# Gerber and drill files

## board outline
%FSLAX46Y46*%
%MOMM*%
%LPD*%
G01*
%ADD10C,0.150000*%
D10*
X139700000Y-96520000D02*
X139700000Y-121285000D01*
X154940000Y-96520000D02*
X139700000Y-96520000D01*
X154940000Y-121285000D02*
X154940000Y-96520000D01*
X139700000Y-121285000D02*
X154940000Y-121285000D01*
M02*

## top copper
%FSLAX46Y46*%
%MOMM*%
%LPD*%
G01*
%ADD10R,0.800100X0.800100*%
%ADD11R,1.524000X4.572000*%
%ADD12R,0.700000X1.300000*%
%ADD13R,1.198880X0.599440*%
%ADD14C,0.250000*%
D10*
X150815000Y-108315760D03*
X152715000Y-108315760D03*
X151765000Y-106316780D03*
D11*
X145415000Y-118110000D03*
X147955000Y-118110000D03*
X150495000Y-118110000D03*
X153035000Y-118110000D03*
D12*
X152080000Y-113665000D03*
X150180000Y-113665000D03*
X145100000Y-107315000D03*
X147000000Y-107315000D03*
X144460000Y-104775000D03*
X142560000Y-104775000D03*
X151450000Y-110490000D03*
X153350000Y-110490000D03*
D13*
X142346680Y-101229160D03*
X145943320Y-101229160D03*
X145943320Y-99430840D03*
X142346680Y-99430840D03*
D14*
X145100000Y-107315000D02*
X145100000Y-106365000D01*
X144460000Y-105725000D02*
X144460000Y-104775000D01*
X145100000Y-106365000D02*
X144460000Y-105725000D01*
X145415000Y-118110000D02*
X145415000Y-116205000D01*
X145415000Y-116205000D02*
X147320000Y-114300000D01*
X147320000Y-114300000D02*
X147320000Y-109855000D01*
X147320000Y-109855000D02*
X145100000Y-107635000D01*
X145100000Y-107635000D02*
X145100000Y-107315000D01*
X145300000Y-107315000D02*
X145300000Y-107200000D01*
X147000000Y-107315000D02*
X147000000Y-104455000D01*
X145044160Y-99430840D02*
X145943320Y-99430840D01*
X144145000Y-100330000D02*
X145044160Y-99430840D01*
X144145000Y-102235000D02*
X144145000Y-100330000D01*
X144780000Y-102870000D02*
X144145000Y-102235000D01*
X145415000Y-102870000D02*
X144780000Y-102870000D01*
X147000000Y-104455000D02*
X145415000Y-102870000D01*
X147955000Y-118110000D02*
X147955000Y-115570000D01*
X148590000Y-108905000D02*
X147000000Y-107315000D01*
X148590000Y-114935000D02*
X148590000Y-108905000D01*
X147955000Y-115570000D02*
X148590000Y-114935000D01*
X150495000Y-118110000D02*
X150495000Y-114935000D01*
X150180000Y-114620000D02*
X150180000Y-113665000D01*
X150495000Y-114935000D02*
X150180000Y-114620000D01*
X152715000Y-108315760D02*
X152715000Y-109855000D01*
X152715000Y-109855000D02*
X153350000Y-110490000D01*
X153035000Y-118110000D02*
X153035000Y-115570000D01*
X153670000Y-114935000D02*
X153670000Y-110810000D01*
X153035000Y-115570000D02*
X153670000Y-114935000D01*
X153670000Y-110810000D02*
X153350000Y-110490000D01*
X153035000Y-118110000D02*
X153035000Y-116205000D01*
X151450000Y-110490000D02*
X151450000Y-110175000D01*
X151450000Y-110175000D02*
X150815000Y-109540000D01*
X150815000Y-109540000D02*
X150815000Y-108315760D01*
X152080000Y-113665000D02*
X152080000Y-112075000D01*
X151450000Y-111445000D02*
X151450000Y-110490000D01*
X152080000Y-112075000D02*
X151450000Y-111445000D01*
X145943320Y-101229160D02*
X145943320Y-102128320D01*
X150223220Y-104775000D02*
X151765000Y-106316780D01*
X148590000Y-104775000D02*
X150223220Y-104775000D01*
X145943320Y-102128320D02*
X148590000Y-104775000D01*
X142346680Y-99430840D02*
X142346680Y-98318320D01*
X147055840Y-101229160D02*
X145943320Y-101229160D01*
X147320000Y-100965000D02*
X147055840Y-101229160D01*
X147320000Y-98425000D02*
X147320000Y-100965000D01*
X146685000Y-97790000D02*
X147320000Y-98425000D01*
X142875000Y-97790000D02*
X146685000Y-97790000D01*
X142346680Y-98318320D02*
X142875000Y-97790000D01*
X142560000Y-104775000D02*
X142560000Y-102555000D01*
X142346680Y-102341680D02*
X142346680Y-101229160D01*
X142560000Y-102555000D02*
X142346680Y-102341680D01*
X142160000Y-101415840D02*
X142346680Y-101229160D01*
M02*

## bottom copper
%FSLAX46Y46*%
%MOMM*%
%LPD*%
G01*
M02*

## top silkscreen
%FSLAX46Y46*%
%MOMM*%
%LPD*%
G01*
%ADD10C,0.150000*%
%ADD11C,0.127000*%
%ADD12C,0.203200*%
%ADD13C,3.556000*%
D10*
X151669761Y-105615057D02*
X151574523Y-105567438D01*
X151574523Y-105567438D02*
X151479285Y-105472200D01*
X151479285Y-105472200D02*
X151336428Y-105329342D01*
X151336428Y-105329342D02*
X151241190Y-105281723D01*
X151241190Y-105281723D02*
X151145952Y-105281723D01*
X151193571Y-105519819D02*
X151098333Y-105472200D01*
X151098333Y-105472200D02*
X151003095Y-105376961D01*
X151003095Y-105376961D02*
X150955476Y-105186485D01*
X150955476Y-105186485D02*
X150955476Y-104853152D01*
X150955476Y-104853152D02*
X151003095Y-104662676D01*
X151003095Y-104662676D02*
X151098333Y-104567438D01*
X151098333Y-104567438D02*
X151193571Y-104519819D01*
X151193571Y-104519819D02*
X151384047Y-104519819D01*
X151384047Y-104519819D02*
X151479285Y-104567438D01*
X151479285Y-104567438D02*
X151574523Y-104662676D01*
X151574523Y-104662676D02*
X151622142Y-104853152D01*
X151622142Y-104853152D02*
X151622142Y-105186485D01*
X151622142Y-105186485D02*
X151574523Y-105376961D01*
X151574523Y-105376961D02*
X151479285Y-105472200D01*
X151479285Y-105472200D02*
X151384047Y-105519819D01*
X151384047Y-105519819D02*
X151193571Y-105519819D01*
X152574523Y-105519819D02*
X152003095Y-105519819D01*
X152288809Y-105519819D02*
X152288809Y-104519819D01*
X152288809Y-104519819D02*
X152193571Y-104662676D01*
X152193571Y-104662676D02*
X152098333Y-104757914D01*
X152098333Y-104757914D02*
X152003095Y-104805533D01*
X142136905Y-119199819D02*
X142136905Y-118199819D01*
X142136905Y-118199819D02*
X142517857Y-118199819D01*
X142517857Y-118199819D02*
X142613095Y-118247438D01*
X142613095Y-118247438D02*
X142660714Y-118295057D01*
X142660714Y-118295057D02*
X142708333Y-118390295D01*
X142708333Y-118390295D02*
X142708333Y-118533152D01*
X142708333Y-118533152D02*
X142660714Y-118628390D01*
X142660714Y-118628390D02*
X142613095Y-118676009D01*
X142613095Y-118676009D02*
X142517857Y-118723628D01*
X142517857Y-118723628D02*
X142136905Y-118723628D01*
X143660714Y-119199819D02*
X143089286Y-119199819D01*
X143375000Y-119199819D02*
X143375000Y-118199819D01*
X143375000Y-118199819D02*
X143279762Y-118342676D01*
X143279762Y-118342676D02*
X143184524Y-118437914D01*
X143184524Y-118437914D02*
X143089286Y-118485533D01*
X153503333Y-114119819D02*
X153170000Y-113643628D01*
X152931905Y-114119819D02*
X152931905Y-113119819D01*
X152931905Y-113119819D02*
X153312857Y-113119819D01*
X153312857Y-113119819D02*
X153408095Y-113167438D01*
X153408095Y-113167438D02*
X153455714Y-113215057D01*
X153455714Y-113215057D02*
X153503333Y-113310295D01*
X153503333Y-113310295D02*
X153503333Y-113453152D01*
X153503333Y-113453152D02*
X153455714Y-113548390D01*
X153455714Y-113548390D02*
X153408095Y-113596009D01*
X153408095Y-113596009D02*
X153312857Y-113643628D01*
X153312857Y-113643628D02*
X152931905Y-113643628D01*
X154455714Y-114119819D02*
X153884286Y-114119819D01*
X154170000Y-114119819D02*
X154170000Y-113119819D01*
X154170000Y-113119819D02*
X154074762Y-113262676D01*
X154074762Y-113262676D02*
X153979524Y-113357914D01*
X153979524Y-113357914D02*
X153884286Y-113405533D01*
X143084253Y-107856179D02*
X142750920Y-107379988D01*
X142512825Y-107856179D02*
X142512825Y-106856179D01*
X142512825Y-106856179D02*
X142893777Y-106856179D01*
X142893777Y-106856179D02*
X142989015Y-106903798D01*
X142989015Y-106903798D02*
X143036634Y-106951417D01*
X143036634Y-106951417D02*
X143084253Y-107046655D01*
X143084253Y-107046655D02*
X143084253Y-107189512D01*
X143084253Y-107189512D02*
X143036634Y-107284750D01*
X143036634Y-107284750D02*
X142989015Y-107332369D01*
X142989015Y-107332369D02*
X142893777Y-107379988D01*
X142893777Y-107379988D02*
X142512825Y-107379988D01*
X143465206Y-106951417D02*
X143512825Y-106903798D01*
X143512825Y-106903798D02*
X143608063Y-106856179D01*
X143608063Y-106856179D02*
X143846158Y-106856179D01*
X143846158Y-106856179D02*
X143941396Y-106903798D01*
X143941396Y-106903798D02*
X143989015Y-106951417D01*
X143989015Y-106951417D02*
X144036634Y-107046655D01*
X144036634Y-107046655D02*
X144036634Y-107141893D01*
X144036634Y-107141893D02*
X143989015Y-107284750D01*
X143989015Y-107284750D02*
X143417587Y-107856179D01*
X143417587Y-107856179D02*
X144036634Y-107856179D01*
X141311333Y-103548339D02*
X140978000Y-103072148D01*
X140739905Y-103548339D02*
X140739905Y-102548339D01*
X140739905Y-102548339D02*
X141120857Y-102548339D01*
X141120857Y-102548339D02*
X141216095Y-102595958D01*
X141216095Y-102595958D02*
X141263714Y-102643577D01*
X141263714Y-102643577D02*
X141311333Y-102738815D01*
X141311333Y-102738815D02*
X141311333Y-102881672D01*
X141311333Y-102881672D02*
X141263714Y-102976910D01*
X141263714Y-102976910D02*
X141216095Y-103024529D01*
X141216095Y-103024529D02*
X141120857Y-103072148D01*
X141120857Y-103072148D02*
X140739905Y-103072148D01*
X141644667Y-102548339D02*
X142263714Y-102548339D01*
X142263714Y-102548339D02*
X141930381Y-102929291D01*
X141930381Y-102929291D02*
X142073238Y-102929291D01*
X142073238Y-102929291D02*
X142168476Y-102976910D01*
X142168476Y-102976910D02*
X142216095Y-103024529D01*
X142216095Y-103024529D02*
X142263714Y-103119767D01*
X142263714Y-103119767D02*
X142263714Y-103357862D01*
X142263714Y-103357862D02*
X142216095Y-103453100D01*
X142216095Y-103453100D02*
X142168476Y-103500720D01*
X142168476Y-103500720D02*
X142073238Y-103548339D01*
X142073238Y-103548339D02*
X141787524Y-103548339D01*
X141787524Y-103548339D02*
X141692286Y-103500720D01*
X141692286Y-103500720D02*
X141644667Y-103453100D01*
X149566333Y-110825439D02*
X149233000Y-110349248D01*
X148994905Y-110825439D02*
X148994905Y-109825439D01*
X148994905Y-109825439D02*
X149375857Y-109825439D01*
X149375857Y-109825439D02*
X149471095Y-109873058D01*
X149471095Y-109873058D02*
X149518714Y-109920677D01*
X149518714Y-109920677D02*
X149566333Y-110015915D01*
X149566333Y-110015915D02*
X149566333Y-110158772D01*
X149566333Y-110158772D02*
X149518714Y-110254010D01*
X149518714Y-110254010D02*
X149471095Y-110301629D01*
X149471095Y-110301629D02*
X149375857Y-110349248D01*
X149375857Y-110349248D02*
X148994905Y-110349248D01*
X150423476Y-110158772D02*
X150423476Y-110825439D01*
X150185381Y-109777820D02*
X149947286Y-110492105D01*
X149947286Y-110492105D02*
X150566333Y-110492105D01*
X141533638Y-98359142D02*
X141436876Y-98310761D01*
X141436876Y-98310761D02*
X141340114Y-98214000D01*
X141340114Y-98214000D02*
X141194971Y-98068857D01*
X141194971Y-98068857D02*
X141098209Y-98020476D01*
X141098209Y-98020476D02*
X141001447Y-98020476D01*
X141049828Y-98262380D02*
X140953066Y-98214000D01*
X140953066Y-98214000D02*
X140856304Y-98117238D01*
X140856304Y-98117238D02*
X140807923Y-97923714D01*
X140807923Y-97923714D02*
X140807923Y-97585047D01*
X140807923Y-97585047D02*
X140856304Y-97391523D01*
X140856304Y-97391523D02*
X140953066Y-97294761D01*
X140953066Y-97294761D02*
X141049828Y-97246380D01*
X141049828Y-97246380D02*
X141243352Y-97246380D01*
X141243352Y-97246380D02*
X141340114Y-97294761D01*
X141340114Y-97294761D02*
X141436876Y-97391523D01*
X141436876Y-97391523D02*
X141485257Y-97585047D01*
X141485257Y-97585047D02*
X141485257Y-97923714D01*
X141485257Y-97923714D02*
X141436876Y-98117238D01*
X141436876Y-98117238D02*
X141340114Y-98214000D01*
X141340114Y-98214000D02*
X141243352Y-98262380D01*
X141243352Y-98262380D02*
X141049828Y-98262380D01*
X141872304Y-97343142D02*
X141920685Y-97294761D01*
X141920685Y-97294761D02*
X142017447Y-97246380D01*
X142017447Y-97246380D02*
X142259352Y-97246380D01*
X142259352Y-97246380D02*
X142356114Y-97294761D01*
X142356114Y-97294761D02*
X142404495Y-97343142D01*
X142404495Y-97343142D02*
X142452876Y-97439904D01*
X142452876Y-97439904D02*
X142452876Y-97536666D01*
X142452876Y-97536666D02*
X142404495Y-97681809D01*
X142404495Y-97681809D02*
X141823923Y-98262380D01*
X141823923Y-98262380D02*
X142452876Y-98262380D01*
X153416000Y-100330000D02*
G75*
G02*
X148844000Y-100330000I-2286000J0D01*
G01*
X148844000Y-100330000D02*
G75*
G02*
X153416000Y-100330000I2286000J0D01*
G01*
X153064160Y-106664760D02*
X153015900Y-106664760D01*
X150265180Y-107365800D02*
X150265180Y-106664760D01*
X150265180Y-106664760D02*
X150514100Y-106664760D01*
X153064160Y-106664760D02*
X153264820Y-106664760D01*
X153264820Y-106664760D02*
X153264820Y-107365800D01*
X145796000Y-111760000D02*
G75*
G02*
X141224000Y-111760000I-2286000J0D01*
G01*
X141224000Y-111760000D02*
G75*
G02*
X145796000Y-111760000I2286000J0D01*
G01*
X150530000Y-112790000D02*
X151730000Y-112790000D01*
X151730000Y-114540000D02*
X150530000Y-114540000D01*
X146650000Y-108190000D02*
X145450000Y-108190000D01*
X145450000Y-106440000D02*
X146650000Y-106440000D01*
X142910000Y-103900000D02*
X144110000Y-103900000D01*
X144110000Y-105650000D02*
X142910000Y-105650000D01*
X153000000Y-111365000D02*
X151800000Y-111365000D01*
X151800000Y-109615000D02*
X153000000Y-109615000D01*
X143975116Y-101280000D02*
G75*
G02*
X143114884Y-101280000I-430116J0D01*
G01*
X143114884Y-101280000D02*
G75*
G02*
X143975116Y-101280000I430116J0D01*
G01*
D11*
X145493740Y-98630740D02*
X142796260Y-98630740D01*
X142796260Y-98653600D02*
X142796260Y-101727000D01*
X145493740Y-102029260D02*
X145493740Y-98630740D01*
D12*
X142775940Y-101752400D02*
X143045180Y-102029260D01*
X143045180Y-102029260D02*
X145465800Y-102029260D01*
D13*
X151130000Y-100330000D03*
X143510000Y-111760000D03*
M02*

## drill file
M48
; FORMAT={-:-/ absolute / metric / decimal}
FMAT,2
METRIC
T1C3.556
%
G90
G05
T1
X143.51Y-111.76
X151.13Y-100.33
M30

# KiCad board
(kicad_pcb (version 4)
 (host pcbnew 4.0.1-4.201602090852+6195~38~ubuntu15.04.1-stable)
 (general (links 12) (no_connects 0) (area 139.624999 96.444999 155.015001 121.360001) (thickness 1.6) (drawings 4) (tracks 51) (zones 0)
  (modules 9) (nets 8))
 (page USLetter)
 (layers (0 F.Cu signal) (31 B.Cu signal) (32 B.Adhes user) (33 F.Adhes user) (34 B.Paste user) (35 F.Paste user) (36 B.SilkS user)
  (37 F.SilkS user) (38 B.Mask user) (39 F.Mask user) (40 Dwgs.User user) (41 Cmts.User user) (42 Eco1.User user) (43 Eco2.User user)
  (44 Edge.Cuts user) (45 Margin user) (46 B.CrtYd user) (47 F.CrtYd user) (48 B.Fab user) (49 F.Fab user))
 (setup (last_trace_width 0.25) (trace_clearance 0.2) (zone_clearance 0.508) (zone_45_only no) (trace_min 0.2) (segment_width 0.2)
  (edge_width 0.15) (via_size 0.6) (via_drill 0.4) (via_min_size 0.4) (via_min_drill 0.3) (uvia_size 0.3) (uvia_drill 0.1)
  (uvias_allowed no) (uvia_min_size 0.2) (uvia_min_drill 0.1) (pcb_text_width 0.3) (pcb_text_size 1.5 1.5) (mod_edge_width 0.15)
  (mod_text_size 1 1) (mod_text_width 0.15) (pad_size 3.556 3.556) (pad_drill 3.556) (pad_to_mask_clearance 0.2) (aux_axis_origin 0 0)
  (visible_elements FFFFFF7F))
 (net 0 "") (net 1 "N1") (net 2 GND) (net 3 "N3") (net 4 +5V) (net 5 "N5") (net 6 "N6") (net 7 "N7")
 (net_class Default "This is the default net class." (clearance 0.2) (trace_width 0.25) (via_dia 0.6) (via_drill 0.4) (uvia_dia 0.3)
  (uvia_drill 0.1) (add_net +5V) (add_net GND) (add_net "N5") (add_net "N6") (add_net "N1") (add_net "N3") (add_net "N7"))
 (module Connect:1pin (layer F.Cu) (at 151.13 100.33)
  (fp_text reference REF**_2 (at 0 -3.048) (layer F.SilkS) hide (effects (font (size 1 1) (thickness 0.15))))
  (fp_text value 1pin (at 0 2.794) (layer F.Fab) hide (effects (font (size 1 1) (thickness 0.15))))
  (fp_circle (center 0 0) (end 0 -2.286) (layer F.SilkS) (width 0.15))
  (pad "" np_thru_hole circle (at 0 0) (size 3.556 3.556) (drill 3.556) (layers *.Cu *.Mask F.SilkS)))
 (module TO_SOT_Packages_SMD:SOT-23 (layer F.Cu) (at 151.765 107.315)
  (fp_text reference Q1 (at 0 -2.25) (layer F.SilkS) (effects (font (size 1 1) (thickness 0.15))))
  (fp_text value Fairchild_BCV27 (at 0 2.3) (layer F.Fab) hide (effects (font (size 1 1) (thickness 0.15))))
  (fp_line (start 1.29916 -0.65024) (end 1.2509 -0.65024) (layer F.SilkS) (width 0.15))
  (fp_line (start -1.49982 0.0508) (end -1.49982 -0.65024) (layer F.SilkS) (width 0.15))
  (fp_line (start -1.49982 -0.65024) (end -1.2509 -0.65024) (layer F.SilkS) (width 0.15))
  (fp_line (start 1.29916 -0.65024) (end 1.49982 -0.65024) (layer F.SilkS) (width 0.15))
  (fp_line (start 1.49982 -0.65024) (end 1.49982 0.0508) (layer F.SilkS) (width 0.15))
  (pad 1 smd rect (at -0.95 1.00076) (size 0.8001 0.8001) (layers F.Cu F.Paste F.Mask) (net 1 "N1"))
  (pad 2 smd rect (at 0.95 1.00076) (size 0.8001 0.8001) (layers F.Cu F.Paste F.Mask) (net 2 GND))
  (pad 3 smd rect (at 0 -0.99822) (size 0.8001 0.8001) (layers F.Cu F.Paste F.Mask) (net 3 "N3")))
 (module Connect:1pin (layer F.Cu) (at 143.51 111.76)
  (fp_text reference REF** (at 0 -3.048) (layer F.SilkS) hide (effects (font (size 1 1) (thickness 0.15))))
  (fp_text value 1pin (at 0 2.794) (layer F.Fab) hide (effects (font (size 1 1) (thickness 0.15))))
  (fp_circle (center 0 0) (end 0 -2.286) (layer F.SilkS) (width 0.15))
  (pad "" np_thru_hole circle (at 0 0) (size 3.556 3.556) (drill 3.556) (layers *.Cu *.Mask F.SilkS)))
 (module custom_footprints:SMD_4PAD (layer F.Cu) (at 149.225 116.84)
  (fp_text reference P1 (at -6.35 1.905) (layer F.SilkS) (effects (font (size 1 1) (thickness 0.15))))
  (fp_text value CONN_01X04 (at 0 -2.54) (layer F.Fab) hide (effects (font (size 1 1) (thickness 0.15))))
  (pad 1 smd rect (at -3.81 1.27) (size 1.524 4.572) (layers F.Cu F.Paste F.Mask) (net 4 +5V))
  (pad 2 smd rect (at -1.27 1.27) (size 1.524 4.572) (layers F.Cu F.Paste F.Mask) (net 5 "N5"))
  (pad 3 smd rect (at 1.27 1.27) (size 1.524 4.572) (layers F.Cu F.Paste F.Mask) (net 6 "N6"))
  (pad 4 smd rect (at 3.81 1.27) (size 1.524 4.572) (layers F.Cu F.Paste F.Mask) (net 2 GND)))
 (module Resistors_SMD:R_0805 (layer F.Cu) (at 151.13 113.665 180)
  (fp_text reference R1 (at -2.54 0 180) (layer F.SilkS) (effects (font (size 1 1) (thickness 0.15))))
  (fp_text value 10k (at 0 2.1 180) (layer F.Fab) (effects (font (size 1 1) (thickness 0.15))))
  (fp_line (start 0.6 0.875) (end -0.6 0.875) (layer F.SilkS) (width 0.15))
  (fp_line (start -0.6 -0.875) (end 0.6 -0.875) (layer F.SilkS) (width 0.15))
  (pad 1 smd rect (at -0.95 0 180) (size 0.7 1.3) (layers F.Cu F.Paste F.Mask) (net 1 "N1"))
  (pad 2 smd rect (at 0.95 0 180) (size 0.7 1.3) (layers F.Cu F.Paste F.Mask) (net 6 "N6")))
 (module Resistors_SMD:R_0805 (layer F.Cu) (at 146.05 107.315)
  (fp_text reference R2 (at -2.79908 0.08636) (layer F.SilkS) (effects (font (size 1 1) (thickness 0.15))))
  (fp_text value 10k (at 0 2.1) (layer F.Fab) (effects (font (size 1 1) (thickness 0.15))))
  (fp_line (start 0.6 0.875) (end -0.6 0.875) (layer F.SilkS) (width 0.15))
  (fp_line (start -0.6 -0.875) (end 0.6 -0.875) (layer F.SilkS) (width 0.15))
  (pad 1 smd rect (at -0.95 0) (size 0.7 1.3) (layers F.Cu F.Paste F.Mask) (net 4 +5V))
  (pad 2 smd rect (at 0.95 0) (size 0.7 1.3) (layers F.Cu F.Paste F.Mask) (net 5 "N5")))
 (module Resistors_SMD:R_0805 (layer F.Cu) (at 143.51 104.775 180)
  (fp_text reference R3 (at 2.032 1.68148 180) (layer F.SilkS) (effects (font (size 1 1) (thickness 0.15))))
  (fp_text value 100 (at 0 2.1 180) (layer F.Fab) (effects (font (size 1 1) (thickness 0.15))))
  (fp_line (start 0.6 0.875) (end -0.6 0.875) (layer F.SilkS) (width 0.15))
  (fp_line (start -0.6 -0.875) (end 0.6 -0.875) (layer F.SilkS) (width 0.15))
  (pad 1 smd rect (at -0.95 0 180) (size 0.7 1.3) (layers F.Cu F.Paste F.Mask) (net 4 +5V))
  (pad 2 smd rect (at 0.95 0 180) (size 0.7 1.3) (layers F.Cu F.Paste F.Mask) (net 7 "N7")))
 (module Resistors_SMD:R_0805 (layer F.Cu) (at 152.4 110.49)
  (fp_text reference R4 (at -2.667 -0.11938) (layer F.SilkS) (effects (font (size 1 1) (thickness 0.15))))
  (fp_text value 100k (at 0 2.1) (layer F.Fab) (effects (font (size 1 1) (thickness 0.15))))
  (fp_line (start 0.6 0.875) (end -0.6 0.875) (layer F.SilkS) (width 0.15))
  (fp_line (start -0.6 -0.875) (end 0.6 -0.875) (layer F.SilkS) (width 0.15))
  (pad 1 smd rect (at -0.95 0) (size 0.7 1.3) (layers F.Cu F.Paste F.Mask) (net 1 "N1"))
  (pad 2 smd rect (at 0.95 0) (size 0.7 1.3) (layers F.Cu F.Paste F.Mask) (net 2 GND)))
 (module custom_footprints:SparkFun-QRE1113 (layer F.Cu) (at 144.145 100.33)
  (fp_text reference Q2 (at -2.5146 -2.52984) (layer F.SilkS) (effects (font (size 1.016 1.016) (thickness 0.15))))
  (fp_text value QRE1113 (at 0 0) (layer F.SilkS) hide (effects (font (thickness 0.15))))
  (fp_circle (center -0.6 0.95) (end -0.25 0.7) (layer F.SilkS) (width 0.15))
  (fp_line (start 1.34874 -1.69926) (end -1.34874 -1.69926) (layer F.SilkS) (width 0.127))
  (fp_line (start -1.34874 -1.6764) (end -1.34874 1.397) (layer F.SilkS) (width 0.127))
  (fp_line (start 1.34874 1.69926) (end 1.34874 -1.69926) (layer F.SilkS) (width 0.127))
  (fp_line (start -1.36906 1.4224) (end -1.09982 1.69926) (layer F.SilkS) (width 0.2032))
  (fp_line (start -1.09982 1.69926) (end 1.3208 1.69926) (layer F.SilkS) (width 0.2032))
  (pad 1 smd rect (at -1.79832 0.89916) (size 1.19888 0.59944) (layers F.Cu F.Paste F.Mask) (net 7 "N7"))
  (pad 2 smd rect (at 1.79832 0.89916) (size 1.19888 0.59944) (layers F.Cu F.Paste F.Mask) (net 3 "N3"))
  (pad 3 smd rect (at 1.79832 -0.89916) (size 1.19888 0.59944) (layers F.Cu F.Paste F.Mask) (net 5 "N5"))
  (pad 4 smd rect (at -1.79832 -0.89916) (size 1.19888 0.59944) (layers F.Cu F.Paste F.Mask) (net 3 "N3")))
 (gr_line (start 139.7 96.52) (end 139.7 121.285) (angle 90) (layer Edge.Cuts) (width 0.15))
 (gr_line (start 154.94 96.52) (end 139.7 96.52) (angle 90) (layer Edge.Cuts) (width 0.15))
 (gr_line (start 154.94 121.285) (end 154.94 96.52) (angle 90) (layer Edge.Cuts) (width 0.15))
 (gr_line (start 139.7 121.285) (end 154.94 121.285) (angle 90) (layer Edge.Cuts) (width 0.15))
 (segment (start 145.1 107.315) (end 145.1 106.365) (width 0.25) (layer F.Cu) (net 4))
 (segment (start 144.46 105.725) (end 144.46 104.775) (width 0.25) (layer F.Cu) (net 4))
 (segment (start 145.1 106.365) (end 144.46 105.725) (width 0.25) (layer F.Cu) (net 4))
 (segment (start 145.415 118.11) (end 145.415 116.205) (width 0.25) (layer F.Cu) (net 4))
 (segment (start 145.415 116.205) (end 147.32 114.3) (width 0.25) (layer F.Cu) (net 4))
 (segment (start 147.32 114.3) (end 147.32 109.855) (width 0.25) (layer F.Cu) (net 4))
 (segment (start 147.32 109.855) (end 145.1 107.635) (width 0.25) (layer F.Cu) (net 4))
 (segment (start 145.1 107.635) (end 145.1 107.315) (width 0.25) (layer F.Cu) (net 4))
 (segment (start 145.3 107.315) (end 145.3 107.2) (width 0.25) (layer F.Cu) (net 4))
 (segment (start 147 107.315) (end 147 104.455) (width 0.25) (layer F.Cu) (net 5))
 (segment (start 145.04416 99.43084) (end 145.94332 99.43084) (width 0.25) (layer F.Cu) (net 5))
 (segment (start 144.145 100.33) (end 145.04416 99.43084) (width 0.25) (layer F.Cu) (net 5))
 (segment (start 144.145 102.235) (end 144.145 100.33) (width 0.25) (layer F.Cu) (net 5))
 (segment (start 144.78 102.87) (end 144.145 102.235) (width 0.25) (layer F.Cu) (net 5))
 (segment (start 145.415 102.87) (end 144.78 102.87) (width 0.25) (layer F.Cu) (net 5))
 (segment (start 147 104.455) (end 145.415 102.87) (width 0.25) (layer F.Cu) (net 5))
 (segment (start 147.955 118.11) (end 147.955 115.57) (width 0.25) (layer F.Cu) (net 5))
 (segment (start 148.59 108.905) (end 147 107.315) (width 0.25) (layer F.Cu) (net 5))
 (segment (start 148.59 114.935) (end 148.59 108.905) (width 0.25) (layer F.Cu) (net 5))
 (segment (start 147.955 115.57) (end 148.59 114.935) (width 0.25) (layer F.Cu) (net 5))
 (segment (start 150.495 118.11) (end 150.495 114.935) (width 0.25) (layer F.Cu) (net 6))
 (segment (start 150.18 114.62) (end 150.18 113.665) (width 0.25) (layer F.Cu) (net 6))
 (segment (start 150.495 114.935) (end 150.18 114.62) (width 0.25) (layer F.Cu) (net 6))
 (segment (start 152.715 108.31576) (end 152.715 109.855) (width 0.25) (layer F.Cu) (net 2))
 (segment (start 152.715 109.855) (end 153.35 110.49) (width 0.25) (layer F.Cu) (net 2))
 (segment (start 153.035 118.11) (end 153.035 115.57) (width 0.25) (layer F.Cu) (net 2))
 (segment (start 153.67 114.935) (end 153.67 110.81) (width 0.25) (layer F.Cu) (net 2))
 (segment (start 153.035 115.57) (end 153.67 114.935) (width 0.25) (layer F.Cu) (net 2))
 (segment (start 153.67 110.81) (end 153.35 110.49) (width 0.25) (layer F.Cu) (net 2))
 (segment (start 153.035 118.11) (end 153.035 116.205) (width 0.25) (layer F.Cu) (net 2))
 (segment (start 151.45 110.49) (end 151.45 110.175) (width 0.25) (layer F.Cu) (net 1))
 (segment (start 151.45 110.175) (end 150.815 109.54) (width 0.25) (layer F.Cu) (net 1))
 (segment (start 150.815 109.54) (end 150.815 108.31576) (width 0.25) (layer F.Cu) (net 1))
 (segment (start 152.08 113.665) (end 152.08 112.075) (width 0.25) (layer F.Cu) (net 1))
 (segment (start 151.45 111.445) (end 151.45 110.49) (width 0.25) (layer F.Cu) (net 1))
 (segment (start 152.08 112.075) (end 151.45 111.445) (width 0.25) (layer F.Cu) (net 1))
 (segment (start 145.94332 101.22916) (end 145.94332 102.12832) (width 0.25) (layer F.Cu) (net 3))
 (segment (start 150.22322 104.775) (end 151.765 106.31678) (width 0.25) (layer F.Cu) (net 3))
 (segment (start 148.59 104.775) (end 150.22322 104.775) (width 0.25) (layer F.Cu) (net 3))
 (segment (start 145.94332 102.12832) (end 148.59 104.775) (width 0.25) (layer F.Cu) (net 3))
 (segment (start 142.34668 99.43084) (end 142.34668 98.31832) (width 0.25) (layer F.Cu) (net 3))
 (segment (start 147.05584 101.22916) (end 145.94332 101.22916) (width 0.25) (layer F.Cu) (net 3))
 (segment (start 147.32 100.965) (end 147.05584 101.22916) (width 0.25) (layer F.Cu) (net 3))
 (segment (start 147.32 98.425) (end 147.32 100.965) (width 0.25) (layer F.Cu) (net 3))
 (segment (start 146.685 97.79) (end 147.32 98.425) (width 0.25) (layer F.Cu) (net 3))
 (segment (start 142.875 97.79) (end 146.685 97.79) (width 0.25) (layer F.Cu) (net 3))
 (segment (start 142.34668 98.31832) (end 142.875 97.79) (width 0.25) (layer F.Cu) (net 3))
 (segment (start 142.56 104.775) (end 142.56 102.555) (width 0.25) (layer F.Cu) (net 7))
 (segment (start 142.34668 102.34168) (end 142.34668 101.22916) (width 0.25) (layer F.Cu) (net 7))
 (segment (start 142.56 102.555) (end 142.34668 102.34168) (width 0.25) (layer F.Cu) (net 7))
 (segment (start 142.16 101.41584) (end 142.34668 101.22916) (width 0.25) (layer F.Cu) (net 7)))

